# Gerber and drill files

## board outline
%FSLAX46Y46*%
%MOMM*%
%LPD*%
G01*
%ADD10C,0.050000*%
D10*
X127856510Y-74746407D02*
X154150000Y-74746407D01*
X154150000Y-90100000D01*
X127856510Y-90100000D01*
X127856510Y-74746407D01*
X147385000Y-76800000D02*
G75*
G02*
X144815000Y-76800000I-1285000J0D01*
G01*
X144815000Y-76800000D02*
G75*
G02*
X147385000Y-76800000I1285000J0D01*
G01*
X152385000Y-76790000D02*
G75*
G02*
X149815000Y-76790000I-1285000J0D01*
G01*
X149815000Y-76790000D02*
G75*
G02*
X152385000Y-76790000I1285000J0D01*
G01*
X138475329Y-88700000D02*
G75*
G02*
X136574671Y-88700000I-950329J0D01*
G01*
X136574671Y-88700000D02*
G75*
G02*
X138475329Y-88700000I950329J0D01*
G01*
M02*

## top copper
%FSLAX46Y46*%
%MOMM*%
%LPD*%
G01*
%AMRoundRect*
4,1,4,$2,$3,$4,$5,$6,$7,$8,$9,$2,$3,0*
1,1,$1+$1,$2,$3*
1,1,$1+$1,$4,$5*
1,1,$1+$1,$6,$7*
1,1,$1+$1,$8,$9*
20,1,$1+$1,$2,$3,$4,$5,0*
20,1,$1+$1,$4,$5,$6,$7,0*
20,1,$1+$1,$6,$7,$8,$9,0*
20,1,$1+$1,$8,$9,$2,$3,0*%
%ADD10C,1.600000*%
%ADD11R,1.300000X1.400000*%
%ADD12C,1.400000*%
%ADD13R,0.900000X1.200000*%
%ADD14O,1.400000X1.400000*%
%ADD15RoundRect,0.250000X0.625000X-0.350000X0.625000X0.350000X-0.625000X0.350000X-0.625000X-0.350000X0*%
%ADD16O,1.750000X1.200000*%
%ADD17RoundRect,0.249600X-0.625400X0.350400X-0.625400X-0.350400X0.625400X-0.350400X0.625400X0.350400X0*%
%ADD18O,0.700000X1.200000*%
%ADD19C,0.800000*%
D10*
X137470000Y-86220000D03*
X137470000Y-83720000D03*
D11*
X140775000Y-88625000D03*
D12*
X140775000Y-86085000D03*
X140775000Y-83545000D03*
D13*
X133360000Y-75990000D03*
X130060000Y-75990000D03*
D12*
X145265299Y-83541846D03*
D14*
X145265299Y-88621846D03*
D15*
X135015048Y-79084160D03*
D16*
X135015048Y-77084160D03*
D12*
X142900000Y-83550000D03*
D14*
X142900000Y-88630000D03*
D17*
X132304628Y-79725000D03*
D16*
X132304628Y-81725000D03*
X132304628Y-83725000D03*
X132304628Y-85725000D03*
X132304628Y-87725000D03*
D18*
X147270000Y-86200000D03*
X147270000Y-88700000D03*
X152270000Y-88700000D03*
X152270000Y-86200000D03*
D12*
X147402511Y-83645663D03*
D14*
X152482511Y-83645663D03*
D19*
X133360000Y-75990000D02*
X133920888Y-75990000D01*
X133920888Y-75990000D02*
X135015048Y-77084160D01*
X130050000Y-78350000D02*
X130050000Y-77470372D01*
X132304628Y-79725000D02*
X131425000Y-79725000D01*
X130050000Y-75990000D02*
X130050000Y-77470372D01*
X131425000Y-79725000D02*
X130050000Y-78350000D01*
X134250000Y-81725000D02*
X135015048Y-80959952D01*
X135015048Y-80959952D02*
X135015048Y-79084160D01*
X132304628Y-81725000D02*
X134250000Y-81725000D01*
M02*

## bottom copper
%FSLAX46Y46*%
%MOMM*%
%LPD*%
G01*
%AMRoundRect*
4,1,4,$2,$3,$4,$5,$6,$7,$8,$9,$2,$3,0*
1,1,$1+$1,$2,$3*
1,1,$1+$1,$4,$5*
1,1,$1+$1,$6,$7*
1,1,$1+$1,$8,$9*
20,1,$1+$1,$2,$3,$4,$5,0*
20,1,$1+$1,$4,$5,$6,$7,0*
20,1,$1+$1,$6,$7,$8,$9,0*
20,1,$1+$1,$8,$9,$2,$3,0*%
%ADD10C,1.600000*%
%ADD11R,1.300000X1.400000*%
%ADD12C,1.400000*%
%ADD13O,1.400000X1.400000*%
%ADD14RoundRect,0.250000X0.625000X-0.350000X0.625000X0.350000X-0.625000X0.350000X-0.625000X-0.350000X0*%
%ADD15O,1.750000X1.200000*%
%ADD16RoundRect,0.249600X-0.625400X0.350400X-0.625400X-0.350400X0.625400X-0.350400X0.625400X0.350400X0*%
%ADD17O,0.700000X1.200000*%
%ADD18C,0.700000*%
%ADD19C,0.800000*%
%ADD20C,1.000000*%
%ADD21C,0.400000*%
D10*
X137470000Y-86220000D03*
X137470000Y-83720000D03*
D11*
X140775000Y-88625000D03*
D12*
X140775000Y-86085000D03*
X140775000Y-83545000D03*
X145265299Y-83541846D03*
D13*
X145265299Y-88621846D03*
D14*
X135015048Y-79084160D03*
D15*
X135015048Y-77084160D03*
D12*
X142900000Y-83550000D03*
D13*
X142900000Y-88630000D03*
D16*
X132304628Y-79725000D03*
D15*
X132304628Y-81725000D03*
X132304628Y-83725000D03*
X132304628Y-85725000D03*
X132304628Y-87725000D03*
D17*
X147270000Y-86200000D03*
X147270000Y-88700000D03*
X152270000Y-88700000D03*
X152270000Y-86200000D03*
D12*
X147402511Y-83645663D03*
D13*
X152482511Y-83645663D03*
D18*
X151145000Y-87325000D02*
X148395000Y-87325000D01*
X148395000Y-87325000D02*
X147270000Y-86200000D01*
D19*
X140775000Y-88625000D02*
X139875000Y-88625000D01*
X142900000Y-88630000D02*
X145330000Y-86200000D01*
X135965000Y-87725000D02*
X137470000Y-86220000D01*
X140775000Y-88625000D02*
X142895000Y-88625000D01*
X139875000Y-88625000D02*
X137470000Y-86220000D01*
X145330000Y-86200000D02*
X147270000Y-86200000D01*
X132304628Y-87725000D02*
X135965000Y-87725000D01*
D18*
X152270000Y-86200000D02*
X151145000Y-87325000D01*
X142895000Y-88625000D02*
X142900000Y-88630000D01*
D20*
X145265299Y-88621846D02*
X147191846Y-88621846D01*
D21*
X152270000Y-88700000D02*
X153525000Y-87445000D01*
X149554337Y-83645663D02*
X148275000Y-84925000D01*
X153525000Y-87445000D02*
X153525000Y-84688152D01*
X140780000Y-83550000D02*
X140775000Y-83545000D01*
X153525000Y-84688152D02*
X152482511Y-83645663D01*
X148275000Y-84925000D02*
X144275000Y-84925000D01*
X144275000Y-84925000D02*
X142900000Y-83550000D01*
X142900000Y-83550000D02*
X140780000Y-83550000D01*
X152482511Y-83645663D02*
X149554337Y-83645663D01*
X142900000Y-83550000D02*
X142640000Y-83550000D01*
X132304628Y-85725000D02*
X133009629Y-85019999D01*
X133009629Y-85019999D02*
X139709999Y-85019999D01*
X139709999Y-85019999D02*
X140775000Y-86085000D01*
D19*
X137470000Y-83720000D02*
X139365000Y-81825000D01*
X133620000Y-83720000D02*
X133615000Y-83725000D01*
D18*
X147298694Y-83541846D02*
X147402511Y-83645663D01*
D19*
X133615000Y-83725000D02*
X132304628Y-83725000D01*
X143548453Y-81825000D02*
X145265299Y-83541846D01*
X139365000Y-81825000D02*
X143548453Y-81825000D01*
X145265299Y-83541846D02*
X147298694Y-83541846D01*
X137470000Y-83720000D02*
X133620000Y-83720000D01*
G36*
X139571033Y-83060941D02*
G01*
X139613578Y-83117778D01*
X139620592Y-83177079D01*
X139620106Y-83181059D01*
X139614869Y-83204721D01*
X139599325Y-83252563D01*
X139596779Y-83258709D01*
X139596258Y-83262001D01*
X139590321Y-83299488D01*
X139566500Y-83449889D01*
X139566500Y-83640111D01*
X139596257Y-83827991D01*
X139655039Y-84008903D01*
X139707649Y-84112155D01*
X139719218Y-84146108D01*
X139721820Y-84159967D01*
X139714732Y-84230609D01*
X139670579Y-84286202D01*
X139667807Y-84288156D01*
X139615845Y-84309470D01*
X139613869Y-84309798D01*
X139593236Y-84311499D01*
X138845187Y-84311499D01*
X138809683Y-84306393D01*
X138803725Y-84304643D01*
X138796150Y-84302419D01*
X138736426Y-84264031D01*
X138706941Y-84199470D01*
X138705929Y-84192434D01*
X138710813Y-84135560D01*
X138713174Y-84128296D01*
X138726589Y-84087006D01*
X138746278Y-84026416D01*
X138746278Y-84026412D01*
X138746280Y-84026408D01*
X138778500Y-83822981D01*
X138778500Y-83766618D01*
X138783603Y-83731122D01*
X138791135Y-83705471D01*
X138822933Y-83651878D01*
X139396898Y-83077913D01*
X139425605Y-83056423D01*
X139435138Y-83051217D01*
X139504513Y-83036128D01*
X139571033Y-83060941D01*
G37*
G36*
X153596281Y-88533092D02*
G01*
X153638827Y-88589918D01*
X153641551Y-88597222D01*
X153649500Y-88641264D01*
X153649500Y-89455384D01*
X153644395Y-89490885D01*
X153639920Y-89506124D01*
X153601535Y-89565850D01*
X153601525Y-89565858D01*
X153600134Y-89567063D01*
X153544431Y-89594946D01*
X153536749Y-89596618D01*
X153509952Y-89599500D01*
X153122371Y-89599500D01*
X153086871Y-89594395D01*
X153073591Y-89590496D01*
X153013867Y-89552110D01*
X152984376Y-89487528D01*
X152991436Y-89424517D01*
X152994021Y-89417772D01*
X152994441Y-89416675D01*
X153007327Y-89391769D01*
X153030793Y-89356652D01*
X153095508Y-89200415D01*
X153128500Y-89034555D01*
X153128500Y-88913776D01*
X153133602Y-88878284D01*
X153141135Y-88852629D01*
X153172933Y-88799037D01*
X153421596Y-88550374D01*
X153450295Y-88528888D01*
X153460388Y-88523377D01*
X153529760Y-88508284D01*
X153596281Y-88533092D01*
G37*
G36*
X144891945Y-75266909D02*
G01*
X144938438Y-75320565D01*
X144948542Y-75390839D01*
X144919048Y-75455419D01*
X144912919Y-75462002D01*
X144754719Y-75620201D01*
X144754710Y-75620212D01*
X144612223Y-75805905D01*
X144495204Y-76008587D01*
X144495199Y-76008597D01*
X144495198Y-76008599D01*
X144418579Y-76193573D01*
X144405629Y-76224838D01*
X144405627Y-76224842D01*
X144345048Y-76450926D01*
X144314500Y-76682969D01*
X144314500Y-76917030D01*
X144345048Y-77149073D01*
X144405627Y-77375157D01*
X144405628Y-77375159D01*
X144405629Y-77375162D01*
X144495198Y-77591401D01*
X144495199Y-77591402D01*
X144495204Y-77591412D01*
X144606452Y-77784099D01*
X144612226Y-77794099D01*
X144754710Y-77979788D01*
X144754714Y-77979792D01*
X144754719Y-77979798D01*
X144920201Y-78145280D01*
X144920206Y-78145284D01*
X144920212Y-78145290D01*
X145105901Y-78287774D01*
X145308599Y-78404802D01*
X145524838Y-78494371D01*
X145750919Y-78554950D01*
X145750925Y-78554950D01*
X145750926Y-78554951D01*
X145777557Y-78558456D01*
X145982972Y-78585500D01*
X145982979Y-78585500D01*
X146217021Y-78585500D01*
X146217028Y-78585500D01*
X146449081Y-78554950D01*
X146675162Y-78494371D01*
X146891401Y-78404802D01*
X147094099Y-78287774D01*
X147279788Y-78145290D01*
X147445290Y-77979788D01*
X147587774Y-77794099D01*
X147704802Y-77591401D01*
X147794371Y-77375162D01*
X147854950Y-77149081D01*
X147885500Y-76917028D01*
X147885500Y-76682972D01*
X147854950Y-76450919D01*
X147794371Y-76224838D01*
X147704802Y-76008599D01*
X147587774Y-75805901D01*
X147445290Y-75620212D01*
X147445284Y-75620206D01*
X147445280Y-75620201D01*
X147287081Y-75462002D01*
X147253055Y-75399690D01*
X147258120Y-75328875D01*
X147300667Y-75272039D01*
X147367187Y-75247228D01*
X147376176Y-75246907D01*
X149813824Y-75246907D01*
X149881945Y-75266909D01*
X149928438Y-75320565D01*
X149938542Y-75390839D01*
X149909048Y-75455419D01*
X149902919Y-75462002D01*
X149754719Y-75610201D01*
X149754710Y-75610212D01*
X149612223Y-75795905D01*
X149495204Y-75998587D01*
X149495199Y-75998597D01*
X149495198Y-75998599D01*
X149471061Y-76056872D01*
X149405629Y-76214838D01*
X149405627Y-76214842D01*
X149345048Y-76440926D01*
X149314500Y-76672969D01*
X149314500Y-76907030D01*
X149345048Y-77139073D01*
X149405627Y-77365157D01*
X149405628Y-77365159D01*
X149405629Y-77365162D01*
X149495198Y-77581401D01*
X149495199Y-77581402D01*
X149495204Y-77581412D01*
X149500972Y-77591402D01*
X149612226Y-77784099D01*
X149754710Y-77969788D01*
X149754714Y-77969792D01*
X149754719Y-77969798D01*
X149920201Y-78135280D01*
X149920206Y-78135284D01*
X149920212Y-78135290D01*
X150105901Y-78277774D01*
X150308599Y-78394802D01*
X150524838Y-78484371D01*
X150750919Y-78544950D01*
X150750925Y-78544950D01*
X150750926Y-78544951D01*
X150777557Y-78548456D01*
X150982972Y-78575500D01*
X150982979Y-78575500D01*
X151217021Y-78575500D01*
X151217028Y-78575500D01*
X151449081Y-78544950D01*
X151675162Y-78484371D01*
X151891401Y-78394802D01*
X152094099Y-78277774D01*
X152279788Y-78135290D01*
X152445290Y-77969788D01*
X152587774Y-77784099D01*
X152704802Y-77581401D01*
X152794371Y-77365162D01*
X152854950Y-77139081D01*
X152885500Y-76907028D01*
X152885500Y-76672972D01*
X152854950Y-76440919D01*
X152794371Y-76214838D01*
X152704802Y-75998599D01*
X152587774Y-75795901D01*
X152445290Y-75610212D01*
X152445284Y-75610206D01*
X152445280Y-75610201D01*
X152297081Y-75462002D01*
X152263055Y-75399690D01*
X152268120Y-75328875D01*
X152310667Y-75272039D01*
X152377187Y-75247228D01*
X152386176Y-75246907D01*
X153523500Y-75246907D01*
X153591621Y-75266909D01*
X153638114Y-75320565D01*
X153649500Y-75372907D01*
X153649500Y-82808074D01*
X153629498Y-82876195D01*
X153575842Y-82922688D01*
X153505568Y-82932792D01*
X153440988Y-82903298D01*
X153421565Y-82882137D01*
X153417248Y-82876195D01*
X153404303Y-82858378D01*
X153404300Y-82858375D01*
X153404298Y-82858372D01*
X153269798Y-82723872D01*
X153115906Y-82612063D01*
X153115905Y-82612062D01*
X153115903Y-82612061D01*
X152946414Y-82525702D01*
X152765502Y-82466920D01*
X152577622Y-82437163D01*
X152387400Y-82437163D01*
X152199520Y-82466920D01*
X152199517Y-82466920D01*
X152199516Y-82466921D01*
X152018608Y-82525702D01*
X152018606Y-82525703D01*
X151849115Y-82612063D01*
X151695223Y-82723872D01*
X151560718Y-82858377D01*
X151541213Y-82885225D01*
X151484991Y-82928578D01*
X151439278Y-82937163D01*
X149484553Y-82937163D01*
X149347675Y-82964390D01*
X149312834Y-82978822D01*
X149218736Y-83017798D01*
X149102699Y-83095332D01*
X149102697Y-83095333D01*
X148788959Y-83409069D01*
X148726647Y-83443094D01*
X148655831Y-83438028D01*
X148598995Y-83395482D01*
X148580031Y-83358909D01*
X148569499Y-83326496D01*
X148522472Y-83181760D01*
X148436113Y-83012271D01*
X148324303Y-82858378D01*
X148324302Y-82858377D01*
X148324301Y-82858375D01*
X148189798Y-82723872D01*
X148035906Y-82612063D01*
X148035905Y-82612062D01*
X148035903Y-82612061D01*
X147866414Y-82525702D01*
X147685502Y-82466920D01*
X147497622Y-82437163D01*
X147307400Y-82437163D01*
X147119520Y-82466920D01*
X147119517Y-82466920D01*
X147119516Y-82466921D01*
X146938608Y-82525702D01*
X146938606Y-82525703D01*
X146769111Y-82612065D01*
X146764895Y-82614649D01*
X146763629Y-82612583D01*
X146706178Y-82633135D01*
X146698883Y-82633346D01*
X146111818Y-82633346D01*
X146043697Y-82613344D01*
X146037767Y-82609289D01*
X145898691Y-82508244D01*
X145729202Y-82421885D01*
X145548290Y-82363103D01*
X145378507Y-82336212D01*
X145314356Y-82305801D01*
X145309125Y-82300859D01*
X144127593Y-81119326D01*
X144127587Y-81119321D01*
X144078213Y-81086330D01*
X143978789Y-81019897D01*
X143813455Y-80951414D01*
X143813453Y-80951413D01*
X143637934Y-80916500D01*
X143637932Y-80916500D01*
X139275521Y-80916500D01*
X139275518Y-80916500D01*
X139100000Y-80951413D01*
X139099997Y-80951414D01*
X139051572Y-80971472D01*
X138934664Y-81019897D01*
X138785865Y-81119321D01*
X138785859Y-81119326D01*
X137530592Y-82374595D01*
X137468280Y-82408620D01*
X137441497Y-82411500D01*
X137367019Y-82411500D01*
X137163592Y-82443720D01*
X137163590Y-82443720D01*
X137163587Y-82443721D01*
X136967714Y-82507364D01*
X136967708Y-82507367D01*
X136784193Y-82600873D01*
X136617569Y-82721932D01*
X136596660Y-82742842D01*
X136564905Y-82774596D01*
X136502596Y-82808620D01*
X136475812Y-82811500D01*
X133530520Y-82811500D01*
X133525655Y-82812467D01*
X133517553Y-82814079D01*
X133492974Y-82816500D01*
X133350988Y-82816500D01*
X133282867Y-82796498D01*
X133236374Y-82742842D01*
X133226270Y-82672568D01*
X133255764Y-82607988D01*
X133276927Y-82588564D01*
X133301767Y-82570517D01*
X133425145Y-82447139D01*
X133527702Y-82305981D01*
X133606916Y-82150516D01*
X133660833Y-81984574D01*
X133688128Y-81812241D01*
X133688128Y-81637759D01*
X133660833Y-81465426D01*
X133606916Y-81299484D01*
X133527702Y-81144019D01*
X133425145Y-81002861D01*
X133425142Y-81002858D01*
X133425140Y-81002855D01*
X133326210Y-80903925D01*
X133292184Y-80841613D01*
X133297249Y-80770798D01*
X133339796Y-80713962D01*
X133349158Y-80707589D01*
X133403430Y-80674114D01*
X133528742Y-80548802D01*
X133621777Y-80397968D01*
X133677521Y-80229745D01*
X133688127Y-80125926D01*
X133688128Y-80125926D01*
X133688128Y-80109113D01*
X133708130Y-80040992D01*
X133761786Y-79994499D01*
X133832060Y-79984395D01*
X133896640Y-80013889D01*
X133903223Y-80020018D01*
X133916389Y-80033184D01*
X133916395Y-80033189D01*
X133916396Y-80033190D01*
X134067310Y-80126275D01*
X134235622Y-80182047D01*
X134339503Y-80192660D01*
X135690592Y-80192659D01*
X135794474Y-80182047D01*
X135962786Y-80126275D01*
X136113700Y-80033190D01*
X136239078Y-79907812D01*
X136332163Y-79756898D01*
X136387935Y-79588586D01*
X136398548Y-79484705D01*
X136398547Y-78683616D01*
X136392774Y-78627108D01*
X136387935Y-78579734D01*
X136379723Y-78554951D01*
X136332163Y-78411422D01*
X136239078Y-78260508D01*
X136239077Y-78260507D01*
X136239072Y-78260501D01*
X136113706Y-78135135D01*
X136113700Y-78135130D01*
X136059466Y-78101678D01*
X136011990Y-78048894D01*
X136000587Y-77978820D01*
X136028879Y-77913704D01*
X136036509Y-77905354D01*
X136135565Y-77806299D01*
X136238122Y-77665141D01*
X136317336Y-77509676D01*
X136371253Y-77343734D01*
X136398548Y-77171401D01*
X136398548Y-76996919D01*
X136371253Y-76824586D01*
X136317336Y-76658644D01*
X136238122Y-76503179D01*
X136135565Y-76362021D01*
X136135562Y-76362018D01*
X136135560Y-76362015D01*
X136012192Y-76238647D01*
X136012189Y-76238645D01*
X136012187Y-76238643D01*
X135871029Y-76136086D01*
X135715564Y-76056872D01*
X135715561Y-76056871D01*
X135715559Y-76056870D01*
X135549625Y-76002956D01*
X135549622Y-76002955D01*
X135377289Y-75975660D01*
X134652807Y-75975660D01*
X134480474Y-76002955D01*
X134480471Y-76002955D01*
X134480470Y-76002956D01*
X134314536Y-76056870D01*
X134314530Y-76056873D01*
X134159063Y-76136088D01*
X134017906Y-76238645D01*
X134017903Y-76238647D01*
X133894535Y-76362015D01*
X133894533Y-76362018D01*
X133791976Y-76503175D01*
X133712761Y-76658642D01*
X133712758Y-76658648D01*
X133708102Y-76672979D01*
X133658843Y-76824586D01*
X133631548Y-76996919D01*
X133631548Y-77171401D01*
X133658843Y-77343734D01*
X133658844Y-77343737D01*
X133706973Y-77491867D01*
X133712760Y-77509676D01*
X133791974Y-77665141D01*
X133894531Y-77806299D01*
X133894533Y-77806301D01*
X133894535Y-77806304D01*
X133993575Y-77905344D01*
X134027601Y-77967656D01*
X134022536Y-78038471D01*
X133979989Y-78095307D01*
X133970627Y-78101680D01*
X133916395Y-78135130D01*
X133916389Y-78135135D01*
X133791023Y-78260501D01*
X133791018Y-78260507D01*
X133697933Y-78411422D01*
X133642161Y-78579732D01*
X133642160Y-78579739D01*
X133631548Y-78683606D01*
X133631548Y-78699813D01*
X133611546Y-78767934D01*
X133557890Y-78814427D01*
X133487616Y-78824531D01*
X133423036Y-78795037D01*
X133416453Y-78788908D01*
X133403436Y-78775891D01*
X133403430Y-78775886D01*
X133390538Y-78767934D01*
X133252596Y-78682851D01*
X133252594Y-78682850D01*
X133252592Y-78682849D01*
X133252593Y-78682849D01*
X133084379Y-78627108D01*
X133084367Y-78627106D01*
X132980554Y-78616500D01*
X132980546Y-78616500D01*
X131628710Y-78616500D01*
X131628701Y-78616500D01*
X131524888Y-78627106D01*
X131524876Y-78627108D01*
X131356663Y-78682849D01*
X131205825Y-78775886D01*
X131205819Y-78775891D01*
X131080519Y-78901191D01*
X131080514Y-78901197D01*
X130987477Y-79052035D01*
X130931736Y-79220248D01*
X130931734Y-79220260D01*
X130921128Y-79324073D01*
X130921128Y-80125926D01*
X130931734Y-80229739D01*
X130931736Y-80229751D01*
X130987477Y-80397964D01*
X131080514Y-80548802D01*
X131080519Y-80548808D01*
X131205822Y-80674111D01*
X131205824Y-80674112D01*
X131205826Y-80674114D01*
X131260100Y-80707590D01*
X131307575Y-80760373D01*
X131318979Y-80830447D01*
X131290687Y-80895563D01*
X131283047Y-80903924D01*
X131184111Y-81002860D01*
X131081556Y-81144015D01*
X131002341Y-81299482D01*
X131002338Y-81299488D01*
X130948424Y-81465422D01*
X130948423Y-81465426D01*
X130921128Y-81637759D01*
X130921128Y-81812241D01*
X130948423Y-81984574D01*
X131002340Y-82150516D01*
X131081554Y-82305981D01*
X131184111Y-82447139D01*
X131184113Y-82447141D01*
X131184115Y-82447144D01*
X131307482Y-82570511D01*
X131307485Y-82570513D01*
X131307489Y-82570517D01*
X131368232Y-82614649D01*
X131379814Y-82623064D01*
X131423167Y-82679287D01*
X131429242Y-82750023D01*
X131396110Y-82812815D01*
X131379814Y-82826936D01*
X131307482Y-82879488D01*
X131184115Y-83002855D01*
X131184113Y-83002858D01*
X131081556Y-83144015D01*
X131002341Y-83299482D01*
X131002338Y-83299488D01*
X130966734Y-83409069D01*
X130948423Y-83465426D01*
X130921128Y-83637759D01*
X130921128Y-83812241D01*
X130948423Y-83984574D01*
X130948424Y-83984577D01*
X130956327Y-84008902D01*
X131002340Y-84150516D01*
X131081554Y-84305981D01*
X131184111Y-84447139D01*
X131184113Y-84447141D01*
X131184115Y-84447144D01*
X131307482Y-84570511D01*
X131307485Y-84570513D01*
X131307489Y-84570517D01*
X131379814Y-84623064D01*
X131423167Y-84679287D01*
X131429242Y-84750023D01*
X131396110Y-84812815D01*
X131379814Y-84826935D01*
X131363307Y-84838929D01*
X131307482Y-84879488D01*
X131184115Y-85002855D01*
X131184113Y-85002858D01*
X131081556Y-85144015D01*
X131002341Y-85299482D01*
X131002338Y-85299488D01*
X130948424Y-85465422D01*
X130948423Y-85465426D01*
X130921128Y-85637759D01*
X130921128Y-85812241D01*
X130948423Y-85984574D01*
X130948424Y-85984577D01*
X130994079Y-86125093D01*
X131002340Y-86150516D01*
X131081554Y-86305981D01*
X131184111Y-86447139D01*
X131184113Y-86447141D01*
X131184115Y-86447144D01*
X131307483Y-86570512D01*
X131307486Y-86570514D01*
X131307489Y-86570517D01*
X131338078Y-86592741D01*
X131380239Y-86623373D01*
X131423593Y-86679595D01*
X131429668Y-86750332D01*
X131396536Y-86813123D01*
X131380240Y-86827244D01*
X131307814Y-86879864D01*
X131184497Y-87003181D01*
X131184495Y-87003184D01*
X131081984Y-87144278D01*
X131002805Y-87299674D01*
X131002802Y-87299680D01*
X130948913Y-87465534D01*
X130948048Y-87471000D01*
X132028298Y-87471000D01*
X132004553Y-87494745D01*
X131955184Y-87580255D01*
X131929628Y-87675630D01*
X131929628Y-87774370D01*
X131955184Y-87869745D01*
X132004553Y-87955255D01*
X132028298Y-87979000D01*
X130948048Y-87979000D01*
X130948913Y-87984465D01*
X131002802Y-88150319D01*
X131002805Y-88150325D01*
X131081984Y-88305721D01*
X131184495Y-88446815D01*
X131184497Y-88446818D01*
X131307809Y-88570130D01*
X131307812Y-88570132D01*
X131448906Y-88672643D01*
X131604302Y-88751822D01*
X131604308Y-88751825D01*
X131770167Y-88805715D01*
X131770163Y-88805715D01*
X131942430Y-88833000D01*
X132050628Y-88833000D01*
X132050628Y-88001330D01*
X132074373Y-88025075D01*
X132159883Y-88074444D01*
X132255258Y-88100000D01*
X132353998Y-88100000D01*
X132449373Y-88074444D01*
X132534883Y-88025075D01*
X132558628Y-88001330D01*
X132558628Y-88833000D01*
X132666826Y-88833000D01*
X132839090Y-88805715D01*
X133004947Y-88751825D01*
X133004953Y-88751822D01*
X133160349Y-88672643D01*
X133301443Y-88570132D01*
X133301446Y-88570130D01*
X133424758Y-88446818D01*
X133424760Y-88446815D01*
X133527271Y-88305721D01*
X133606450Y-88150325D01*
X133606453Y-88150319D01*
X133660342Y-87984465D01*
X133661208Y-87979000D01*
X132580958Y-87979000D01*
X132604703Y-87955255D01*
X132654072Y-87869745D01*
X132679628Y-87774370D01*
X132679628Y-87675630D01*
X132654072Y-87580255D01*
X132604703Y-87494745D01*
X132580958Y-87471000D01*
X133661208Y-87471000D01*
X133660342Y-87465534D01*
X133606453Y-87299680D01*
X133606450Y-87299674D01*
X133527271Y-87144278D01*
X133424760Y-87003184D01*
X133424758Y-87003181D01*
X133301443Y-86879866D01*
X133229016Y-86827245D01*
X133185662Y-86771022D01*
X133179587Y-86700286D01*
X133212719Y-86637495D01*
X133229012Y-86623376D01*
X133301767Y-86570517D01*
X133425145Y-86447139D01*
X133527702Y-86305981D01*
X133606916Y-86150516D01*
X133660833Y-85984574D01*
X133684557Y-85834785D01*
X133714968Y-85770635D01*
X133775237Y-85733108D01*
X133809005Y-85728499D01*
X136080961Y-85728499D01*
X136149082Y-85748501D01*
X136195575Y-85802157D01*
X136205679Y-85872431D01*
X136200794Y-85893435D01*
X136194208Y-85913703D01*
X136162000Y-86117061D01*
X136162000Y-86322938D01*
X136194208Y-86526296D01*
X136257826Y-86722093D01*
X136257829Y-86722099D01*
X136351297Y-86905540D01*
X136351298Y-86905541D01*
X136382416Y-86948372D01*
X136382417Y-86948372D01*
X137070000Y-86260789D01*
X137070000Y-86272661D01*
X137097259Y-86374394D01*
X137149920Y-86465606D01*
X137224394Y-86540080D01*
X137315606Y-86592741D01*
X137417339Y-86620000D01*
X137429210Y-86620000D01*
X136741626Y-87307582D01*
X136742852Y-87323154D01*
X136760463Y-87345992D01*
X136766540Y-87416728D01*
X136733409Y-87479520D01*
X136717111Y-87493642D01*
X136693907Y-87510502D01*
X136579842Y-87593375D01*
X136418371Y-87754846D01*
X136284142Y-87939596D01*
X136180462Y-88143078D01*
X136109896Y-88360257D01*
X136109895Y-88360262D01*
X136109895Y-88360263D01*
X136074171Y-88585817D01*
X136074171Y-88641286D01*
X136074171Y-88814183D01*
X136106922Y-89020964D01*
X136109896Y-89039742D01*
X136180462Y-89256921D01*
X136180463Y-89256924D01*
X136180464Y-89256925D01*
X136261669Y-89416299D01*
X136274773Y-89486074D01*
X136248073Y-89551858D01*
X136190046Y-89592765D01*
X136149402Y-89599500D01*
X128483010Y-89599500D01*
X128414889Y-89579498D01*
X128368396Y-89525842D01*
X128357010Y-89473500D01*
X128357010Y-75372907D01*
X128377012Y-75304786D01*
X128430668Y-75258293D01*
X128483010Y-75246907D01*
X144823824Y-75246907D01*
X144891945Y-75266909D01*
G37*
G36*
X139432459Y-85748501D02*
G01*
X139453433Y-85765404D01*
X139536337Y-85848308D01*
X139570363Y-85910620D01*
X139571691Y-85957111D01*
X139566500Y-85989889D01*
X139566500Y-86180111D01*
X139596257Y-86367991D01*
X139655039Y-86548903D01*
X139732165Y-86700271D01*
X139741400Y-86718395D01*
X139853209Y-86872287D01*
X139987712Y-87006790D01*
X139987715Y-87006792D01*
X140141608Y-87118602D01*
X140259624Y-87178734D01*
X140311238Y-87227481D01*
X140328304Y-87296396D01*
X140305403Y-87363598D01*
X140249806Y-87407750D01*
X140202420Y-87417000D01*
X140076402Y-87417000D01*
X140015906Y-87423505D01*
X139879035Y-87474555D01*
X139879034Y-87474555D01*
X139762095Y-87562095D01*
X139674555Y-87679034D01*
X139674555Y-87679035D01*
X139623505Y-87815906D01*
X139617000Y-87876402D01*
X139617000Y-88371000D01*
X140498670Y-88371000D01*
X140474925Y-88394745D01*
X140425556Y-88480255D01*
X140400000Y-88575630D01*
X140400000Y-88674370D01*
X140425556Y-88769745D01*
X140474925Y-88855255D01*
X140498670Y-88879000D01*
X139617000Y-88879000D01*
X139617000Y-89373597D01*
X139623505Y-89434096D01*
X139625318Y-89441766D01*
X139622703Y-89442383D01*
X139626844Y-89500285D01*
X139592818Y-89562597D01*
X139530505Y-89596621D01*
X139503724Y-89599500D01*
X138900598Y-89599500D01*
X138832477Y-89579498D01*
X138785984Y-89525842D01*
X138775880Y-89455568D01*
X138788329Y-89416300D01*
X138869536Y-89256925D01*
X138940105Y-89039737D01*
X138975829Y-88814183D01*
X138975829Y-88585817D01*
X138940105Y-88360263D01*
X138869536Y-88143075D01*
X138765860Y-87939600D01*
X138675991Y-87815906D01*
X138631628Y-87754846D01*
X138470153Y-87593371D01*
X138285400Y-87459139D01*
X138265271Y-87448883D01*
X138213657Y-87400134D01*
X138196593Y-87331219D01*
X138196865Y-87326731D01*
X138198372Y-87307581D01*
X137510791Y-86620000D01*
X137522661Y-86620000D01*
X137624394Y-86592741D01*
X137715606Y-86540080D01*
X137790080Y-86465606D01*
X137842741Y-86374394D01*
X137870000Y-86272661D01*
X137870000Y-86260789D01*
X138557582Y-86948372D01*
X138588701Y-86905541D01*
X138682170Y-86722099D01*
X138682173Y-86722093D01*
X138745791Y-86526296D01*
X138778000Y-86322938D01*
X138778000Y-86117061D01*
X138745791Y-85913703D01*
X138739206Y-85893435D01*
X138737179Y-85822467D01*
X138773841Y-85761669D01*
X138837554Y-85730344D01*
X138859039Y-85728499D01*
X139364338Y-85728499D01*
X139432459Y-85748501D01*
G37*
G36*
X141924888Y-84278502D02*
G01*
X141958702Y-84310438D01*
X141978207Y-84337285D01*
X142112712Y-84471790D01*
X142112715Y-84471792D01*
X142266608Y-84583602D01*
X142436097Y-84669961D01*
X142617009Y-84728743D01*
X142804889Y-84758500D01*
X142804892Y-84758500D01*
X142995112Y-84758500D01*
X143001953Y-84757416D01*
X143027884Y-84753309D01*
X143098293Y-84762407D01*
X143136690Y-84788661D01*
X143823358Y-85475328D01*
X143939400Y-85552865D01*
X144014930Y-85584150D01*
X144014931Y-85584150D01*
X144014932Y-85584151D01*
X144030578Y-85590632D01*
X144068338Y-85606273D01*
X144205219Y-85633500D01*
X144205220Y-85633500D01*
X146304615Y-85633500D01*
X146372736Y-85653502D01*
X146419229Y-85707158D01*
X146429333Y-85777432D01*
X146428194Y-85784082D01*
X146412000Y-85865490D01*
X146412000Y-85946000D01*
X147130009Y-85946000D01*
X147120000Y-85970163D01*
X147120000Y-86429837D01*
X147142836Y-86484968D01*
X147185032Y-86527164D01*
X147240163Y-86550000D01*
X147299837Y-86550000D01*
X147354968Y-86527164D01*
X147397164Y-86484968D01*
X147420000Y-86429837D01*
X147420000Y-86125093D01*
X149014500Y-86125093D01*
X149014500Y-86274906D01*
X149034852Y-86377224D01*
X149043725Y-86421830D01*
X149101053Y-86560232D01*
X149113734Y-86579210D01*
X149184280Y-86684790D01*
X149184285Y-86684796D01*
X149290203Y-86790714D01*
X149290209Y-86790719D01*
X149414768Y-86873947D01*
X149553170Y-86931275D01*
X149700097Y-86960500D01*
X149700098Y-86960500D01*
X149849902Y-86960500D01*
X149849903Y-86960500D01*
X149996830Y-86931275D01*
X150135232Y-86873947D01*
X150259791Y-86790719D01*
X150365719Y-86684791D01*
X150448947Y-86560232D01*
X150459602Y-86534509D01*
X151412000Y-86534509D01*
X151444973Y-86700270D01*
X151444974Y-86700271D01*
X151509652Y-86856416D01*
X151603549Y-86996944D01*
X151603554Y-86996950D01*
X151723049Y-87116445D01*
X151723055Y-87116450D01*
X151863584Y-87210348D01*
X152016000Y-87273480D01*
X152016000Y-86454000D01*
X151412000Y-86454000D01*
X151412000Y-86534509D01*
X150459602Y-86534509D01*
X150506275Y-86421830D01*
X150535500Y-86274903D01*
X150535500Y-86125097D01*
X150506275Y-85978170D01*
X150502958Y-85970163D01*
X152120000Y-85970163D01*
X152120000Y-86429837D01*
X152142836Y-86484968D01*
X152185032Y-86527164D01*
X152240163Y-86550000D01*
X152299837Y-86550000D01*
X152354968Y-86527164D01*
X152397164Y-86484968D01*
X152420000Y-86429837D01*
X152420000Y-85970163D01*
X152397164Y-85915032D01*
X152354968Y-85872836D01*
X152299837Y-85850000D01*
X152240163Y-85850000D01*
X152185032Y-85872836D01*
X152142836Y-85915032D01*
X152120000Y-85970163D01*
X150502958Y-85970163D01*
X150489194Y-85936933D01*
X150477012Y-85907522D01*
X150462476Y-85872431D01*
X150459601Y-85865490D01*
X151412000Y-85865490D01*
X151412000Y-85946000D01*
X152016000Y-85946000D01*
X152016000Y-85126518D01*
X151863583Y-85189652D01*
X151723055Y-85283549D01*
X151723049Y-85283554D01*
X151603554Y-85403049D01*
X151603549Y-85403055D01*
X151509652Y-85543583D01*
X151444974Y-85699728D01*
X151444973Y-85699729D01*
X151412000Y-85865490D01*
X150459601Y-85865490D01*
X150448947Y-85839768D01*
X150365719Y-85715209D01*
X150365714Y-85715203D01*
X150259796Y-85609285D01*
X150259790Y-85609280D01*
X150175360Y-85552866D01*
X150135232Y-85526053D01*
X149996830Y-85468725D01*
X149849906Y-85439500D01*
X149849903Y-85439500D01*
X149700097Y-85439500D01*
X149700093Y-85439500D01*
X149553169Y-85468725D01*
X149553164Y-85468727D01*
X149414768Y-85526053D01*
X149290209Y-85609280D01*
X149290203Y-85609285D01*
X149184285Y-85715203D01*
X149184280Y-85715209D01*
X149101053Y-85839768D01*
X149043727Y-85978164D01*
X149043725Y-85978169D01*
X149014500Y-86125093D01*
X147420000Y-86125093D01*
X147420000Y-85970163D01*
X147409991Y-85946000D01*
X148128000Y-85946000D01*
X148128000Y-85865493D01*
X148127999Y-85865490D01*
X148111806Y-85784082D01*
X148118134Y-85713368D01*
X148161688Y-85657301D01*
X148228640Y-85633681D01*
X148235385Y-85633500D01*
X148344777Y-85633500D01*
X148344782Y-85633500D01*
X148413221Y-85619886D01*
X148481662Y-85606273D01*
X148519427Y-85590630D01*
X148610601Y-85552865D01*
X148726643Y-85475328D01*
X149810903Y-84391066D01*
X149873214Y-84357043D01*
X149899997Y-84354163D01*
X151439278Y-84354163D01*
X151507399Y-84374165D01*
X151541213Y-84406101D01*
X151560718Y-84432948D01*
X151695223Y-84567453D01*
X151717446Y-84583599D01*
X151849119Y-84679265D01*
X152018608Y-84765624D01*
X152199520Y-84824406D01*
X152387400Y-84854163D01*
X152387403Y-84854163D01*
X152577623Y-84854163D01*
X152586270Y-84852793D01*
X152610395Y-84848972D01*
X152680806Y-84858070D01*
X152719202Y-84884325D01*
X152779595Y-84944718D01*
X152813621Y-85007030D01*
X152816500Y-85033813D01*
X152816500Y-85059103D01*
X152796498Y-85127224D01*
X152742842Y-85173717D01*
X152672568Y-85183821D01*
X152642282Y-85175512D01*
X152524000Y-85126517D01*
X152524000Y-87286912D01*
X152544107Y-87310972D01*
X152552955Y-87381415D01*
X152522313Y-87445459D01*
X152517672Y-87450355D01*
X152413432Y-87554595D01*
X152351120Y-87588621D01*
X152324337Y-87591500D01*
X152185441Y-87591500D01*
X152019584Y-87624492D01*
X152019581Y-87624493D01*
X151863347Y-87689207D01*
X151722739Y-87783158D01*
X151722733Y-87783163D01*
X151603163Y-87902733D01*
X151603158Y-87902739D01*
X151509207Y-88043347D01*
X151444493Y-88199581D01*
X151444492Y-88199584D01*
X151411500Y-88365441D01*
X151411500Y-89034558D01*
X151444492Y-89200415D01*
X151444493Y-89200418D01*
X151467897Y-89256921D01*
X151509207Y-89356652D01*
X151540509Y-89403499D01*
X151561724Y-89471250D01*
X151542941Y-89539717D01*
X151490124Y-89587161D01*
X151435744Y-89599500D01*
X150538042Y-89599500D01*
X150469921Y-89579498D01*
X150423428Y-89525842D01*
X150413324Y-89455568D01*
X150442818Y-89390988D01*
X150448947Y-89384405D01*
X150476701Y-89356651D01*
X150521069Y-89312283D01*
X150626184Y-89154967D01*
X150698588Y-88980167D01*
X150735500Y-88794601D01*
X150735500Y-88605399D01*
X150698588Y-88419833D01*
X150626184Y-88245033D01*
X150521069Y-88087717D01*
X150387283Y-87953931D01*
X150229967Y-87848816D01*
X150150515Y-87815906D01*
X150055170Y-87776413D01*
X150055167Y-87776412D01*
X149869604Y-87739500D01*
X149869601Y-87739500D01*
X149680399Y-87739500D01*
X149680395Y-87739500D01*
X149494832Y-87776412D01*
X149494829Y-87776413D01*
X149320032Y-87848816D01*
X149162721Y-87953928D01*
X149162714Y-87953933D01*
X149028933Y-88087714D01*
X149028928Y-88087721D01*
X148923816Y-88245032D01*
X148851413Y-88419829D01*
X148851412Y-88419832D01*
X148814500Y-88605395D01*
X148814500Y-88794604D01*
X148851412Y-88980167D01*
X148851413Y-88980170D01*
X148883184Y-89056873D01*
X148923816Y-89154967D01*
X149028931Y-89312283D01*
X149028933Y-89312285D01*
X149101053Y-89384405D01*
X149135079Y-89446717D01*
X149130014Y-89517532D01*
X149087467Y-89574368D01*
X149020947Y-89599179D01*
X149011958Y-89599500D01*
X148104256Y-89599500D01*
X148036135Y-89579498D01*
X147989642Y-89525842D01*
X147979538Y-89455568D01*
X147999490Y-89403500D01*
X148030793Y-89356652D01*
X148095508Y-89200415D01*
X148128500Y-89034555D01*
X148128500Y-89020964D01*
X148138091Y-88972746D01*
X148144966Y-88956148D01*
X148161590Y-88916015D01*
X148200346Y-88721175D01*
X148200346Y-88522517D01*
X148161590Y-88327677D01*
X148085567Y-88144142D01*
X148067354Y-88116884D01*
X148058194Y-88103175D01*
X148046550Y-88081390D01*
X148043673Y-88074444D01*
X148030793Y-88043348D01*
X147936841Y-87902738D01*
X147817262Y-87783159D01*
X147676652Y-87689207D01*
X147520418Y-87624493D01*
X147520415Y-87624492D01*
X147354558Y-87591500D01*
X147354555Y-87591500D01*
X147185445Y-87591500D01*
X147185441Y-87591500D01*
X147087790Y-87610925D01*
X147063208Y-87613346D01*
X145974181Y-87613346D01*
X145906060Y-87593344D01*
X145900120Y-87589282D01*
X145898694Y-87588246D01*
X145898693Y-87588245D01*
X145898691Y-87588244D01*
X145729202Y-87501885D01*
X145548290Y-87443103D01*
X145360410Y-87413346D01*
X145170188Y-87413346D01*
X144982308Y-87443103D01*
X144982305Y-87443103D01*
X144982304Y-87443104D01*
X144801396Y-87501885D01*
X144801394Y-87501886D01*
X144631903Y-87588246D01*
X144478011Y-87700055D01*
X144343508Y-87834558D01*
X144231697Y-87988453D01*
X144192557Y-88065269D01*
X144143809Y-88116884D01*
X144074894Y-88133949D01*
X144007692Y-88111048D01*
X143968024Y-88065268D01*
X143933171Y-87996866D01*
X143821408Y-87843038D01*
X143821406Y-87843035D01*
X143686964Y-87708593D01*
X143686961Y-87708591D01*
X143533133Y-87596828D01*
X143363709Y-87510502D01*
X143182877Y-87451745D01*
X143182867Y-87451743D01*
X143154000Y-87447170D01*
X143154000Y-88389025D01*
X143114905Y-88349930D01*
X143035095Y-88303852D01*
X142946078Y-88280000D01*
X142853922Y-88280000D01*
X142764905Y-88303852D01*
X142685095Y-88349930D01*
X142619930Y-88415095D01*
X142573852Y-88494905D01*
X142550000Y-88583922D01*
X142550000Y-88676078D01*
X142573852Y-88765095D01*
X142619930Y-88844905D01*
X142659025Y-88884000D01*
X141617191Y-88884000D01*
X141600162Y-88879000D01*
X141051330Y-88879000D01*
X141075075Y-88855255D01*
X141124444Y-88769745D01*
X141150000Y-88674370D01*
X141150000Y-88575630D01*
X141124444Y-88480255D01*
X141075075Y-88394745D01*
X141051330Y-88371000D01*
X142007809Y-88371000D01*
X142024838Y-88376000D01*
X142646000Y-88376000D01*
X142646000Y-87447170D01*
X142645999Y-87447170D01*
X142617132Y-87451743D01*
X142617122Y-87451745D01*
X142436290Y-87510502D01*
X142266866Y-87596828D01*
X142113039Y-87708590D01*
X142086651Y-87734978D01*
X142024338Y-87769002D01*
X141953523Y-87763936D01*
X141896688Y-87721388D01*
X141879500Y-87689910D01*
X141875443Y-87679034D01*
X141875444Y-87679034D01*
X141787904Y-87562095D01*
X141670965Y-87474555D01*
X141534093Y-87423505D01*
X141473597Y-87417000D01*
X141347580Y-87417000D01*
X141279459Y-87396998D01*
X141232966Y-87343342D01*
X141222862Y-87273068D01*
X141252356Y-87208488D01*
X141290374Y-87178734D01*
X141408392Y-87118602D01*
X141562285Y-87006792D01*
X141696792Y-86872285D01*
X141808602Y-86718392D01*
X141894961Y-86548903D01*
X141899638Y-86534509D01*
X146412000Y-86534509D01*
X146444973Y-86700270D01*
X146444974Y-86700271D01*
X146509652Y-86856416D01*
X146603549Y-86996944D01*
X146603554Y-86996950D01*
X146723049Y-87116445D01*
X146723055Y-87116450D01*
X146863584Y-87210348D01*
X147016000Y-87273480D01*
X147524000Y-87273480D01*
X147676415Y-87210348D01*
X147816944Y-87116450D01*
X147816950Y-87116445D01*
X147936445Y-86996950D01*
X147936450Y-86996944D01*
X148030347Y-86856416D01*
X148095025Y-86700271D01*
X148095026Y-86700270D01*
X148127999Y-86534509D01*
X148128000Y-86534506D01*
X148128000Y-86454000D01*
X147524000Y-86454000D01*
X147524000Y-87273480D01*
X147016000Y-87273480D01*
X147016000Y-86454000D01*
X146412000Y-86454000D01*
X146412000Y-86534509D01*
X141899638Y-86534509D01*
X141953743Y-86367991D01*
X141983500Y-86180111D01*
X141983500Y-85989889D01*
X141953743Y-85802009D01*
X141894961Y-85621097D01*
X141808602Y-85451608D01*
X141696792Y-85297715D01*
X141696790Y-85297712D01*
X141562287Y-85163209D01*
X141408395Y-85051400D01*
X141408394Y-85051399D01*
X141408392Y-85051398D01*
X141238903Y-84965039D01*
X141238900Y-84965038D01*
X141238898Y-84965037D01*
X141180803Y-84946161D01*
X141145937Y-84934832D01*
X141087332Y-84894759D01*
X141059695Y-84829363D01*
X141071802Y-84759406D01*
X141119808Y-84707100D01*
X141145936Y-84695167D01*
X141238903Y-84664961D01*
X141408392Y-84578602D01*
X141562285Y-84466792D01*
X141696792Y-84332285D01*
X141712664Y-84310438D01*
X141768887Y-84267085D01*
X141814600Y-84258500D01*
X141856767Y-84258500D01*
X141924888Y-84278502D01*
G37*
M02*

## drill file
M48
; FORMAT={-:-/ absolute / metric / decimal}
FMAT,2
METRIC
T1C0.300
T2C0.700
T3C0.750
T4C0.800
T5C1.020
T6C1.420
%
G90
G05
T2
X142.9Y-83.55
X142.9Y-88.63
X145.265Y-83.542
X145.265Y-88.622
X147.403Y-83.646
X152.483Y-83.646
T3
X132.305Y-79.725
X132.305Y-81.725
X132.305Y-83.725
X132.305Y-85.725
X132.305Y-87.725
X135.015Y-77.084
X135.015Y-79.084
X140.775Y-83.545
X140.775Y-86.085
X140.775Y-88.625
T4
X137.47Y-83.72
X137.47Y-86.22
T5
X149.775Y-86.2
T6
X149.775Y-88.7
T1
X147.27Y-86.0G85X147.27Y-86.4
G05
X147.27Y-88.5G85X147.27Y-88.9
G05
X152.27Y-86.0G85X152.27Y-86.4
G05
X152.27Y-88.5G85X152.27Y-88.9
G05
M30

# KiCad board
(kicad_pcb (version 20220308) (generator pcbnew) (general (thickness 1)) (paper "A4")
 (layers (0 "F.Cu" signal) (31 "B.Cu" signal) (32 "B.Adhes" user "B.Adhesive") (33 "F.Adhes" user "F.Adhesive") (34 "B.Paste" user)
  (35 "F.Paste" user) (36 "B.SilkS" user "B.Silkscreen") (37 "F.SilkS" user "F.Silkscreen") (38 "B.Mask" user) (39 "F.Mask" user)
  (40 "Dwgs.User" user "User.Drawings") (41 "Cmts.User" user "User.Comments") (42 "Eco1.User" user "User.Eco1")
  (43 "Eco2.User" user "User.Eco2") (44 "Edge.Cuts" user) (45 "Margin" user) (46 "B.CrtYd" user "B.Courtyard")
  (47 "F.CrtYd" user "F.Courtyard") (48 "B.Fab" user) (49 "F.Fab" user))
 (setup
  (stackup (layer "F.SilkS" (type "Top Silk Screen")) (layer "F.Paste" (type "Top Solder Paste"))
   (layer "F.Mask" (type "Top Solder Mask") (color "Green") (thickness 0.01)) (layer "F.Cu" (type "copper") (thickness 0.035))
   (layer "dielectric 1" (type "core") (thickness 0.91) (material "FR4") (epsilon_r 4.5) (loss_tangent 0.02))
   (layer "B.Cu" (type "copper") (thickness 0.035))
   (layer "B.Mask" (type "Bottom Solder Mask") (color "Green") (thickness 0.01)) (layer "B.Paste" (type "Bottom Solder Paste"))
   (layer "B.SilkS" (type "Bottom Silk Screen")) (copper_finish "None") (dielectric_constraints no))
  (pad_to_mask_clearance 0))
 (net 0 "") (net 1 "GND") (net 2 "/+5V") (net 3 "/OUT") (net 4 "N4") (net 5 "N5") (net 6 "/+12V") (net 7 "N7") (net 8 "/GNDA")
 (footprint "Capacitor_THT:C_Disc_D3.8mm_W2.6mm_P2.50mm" (layer "F.Cu") (at 137.47 86.22 90)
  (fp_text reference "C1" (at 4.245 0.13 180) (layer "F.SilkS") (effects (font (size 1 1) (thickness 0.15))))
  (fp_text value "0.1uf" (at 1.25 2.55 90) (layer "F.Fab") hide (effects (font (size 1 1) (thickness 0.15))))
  (pad "1" thru_hole circle locked (at 0 0 90) (size 1.6 1.6) (drill 0.8) (layers *.Cu *.Mask) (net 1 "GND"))
  (pad "2" thru_hole circle locked (at 2.5 0 90) (size 1.6 1.6) (drill 0.8) (layers *.Cu *.Mask) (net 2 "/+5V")))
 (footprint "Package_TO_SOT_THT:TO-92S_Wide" (layer "F.Cu") (at 140.775 88.625 90)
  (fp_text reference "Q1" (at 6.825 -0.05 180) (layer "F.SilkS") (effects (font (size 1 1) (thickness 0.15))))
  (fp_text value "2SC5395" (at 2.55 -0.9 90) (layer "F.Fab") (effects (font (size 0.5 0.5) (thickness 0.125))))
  (pad "1" thru_hole rect locked (at 0 0 90) (size 1.4 1.3) (drill 0.75) (layers *.Cu *.Mask) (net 1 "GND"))
  (pad "2" thru_hole circle locked (at 2.54 0 90) (size 1.4 1.4) (drill 0.75) (layers *.Cu *.Mask) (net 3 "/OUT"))
  (pad "3" thru_hole circle locked (at 5.08 0 90) (size 1.4 1.4) (drill 0.75) (layers *.Cu *.Mask) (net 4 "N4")))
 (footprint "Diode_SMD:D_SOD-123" (layer "F.Cu") (at 131.71 75.99 180)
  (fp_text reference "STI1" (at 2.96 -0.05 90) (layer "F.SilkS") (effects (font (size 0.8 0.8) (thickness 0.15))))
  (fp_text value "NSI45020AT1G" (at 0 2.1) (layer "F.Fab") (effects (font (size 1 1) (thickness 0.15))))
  (pad "1" smd rect locked (at -1.65 0 180) (size 0.9 1.2) (layers "F.Cu" "F.Paste" "F.Mask") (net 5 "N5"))
  (pad "2" smd rect locked (at 1.65 0 180) (size 0.9 1.2) (layers "F.Cu" "F.Paste" "F.Mask") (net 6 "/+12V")))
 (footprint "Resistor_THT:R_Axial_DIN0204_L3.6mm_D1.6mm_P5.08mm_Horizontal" (layer "F.Cu") (at 145.265299 83.541846 -90)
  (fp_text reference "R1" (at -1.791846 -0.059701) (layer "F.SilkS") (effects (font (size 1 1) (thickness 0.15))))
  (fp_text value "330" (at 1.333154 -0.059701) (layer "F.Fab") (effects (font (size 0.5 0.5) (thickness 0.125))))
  (pad "1" thru_hole circle locked (at 0 0 270) (size 1.4 1.4) (drill 0.7) (layers *.Cu *.Mask) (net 2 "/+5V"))
  (pad "2" thru_hole oval locked (at 5.08 0 270) (size 1.4 1.4) (drill 0.7) (layers *.Cu *.Mask) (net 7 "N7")))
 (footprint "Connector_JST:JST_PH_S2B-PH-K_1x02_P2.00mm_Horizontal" (layer "F.Cu") (at 135.015048 79.08416 90)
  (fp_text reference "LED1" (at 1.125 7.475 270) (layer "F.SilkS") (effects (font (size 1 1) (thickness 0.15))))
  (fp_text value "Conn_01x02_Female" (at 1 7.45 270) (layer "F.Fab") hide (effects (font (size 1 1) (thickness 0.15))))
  (pad "1" thru_hole roundrect locked (at 0 0 90) (size 1.2 1.75) (drill 0.75) (layers *.Cu *.Mask) (roundrect_rratio 0.2083333333)
   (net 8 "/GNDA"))
  (pad "2" thru_hole oval locked (at 2 0 90) (size 1.2 1.75) (drill 0.75) (layers *.Cu *.Mask) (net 5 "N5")))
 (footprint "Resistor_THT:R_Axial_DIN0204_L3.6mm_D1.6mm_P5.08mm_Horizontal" (layer "F.Cu") (at 142.9 83.55 -90)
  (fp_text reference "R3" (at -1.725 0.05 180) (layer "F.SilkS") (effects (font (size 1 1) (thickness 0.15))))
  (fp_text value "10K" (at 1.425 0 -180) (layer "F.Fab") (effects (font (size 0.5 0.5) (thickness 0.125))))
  (pad "1" thru_hole circle locked (at 0 0 270) (size 1.4 1.4) (drill 0.7) (layers *.Cu *.Mask) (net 4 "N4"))
  (pad "2" thru_hole oval locked (at 5.08 0 270) (size 1.4 1.4) (drill 0.7) (layers *.Cu *.Mask) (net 1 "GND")))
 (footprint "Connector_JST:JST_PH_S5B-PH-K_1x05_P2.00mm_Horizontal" (layer "F.Cu") (at 132.304628 79.725 -90)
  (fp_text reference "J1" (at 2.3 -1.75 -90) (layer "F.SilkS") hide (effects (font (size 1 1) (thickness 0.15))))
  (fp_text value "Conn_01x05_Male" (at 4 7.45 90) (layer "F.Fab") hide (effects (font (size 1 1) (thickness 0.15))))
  (pad "1" thru_hole roundrect locked (at 0 0 270) (size 1.2 1.75) (drill 0.75) (layers *.Cu *.Mask) (roundrect_rratio 0.208)
   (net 6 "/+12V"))
  (pad "2" thru_hole oval locked (at 2 0 270) (size 1.2 1.75) (drill 0.75) (layers *.Cu *.Mask) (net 8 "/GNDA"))
  (pad "3" thru_hole oval locked (at 4 0 270) (size 1.2 1.75) (drill 0.75) (layers *.Cu *.Mask) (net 2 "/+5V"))
  (pad "4" thru_hole oval locked (at 6 0 270) (size 1.2 1.75) (drill 0.75) (layers *.Cu *.Mask) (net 3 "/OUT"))
  (pad "5" thru_hole oval locked (at 8 0 270) (size 1.2 1.75) (drill 0.75) (layers *.Cu *.Mask) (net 1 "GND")))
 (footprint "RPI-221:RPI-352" (layer "F.Cu") (at 146.5 89.6)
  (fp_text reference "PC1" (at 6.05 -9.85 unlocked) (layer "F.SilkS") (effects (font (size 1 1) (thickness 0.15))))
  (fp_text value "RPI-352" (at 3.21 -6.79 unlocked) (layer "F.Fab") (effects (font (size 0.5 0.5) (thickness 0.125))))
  (pad "" np_thru_hole circle (at 3.275 -3.4) (size 1.02 1.02) (drill 1.02) (layers *.Mask))
  (pad "" np_thru_hole circle (at 3.275 -0.9) (size 1.42 1.42) (drill 1.42) (layers *.Mask))
  (pad "1" thru_hole oval (at 0.77 -3.4) (size 0.7 1.2) (drill oval 0.3 0.7) (layers *.Cu *.Mask) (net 1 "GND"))
  (pad "2" thru_hole oval (at 0.77 -0.9) (size 0.7 1.2) (drill oval 0.3 0.7) (layers *.Cu *.Mask) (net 7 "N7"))
  (pad "3" thru_hole oval (at 5.77 -0.9) (size 0.7 1.2) (drill oval 0.3 0.7) (layers *.Cu *.Mask) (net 4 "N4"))
  (pad "4" thru_hole oval (at 5.77 -3.4) (size 0.7 1.2) (drill oval 0.3 0.7) (layers *.Cu *.Mask) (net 1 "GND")))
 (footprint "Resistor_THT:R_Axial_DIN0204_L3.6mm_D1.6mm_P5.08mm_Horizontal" (layer "F.Cu") (at 147.402511 83.645663)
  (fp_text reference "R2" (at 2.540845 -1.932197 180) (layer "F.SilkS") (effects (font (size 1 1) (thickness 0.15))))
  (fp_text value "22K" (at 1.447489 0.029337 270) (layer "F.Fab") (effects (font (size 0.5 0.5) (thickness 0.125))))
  (pad "1" thru_hole circle locked (at 0 0) (size 1.4 1.4) (drill 0.7) (layers *.Cu *.Mask) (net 2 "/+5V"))
  (pad "2" thru_hole oval locked (at 5.08 0) (size 1.4 1.4) (drill 0.7) (layers *.Cu *.Mask) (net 4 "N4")))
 (gr_rect (start 127.85651 74.746407) (end 154.15 90.1) (stroke (width 0.05) (type solid)) (fill none) (layer "Edge.Cuts"))
 (gr_circle (center 146.1 76.8) (end 147.385 76.8) (stroke (width 0.05) (type solid)) (fill none) (layer "Edge.Cuts"))
 (gr_circle (center 151.1 76.79) (end 152.385 76.79) (stroke (width 0.05) (type solid)) (fill none) (layer "Edge.Cuts"))
 (gr_circle (center 137.525 88.7) (end 138.475 88.675) (stroke (width 0.05) (type solid)) (fill none) (layer "Edge.Cuts"))
 (segment (start 151.145 87.325) (end 148.395 87.325) (width 0.7) (layer "B.Cu") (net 1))
 (segment (start 148.395 87.325) (end 147.27 86.2) (width 0.7) (layer "B.Cu") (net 1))
 (segment (start 140.775 88.625) (end 139.875 88.625) (width 0.8) (layer "B.Cu") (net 1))
 (segment (start 142.9 88.63) (end 145.33 86.2) (width 0.8) (layer "B.Cu") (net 1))
 (segment (start 135.965 87.725) (end 137.47 86.22) (width 0.8) (layer "B.Cu") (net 1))
 (segment (start 140.775 88.625) (end 142.895 88.625) (width 0.8) (layer "B.Cu") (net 1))
 (segment (start 139.875 88.625) (end 137.47 86.22) (width 0.8) (layer "B.Cu") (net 1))
 (segment (start 145.33 86.2) (end 147.27 86.2) (width 0.8) (layer "B.Cu") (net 1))
 (segment (start 132.304628 87.725) (end 135.965 87.725) (width 0.8) (layer "B.Cu") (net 1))
 (segment (start 152.27 86.2) (end 151.145 87.325) (width 0.7) (layer "B.Cu") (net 1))
 (segment (start 142.895 88.625) (end 142.9 88.63) (width 0.7) (layer "B.Cu") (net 1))
 (segment (start 133.36 75.99) (end 133.920888 75.99) (width 0.8) (layer "F.Cu") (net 5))
 (segment (start 133.920888 75.99) (end 135.015048 77.08416) (width 0.8) (layer "F.Cu") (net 5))
 (segment (start 145.265299 88.621846) (end 147.191846 88.621846) (width 1) (layer "B.Cu") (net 7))
 (segment (start 152.27 88.7) (end 153.525 87.445) (width 0.4) (layer "B.Cu") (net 4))
 (segment (start 149.554337 83.645663) (end 148.275 84.925) (width 0.4) (layer "B.Cu") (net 4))
 (segment (start 153.525 87.445) (end 153.525 84.688152) (width 0.4) (layer "B.Cu") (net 4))
 (segment (start 140.78 83.55) (end 140.775 83.545) (width 0.4) (layer "B.Cu") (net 4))
 (segment (start 153.525 84.688152) (end 152.482511 83.645663) (width 0.4) (layer "B.Cu") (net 4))
 (segment (start 148.275 84.925) (end 144.275 84.925) (width 0.4) (layer "B.Cu") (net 4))
 (segment (start 144.275 84.925) (end 142.9 83.55) (width 0.4) (layer "B.Cu") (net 4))
 (segment (start 142.9 83.55) (end 140.78 83.55) (width 0.4) (layer "B.Cu") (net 4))
 (segment (start 152.482511 83.645663) (end 149.554337 83.645663) (width 0.4) (layer "B.Cu") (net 4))
 (segment (start 142.9 83.55) (end 142.64 83.55) (width 0.4) (layer "B.Cu") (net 4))
 (segment (start 132.304628 85.725) (end 133.009629 85.019999) (width 0.4) (layer "B.Cu") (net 3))
 (segment (start 133.009629 85.019999) (end 139.709999 85.019999) (width 0.4) (layer "B.Cu") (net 3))
 (segment (start 139.709999 85.019999) (end 140.775 86.085) (width 0.4) (layer "B.Cu") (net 3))
 (segment (start 130.05 78.35) (end 130.05 77.470372) (width 0.8) (layer "F.Cu") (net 6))
 (segment (start 132.304628 79.725) (end 131.425 79.725) (width 0.8) (layer "F.Cu") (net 6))
 (segment (start 130.05 75.99) (end 130.05 77.470372) (width 0.8) (layer "F.Cu") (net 6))
 (segment (start 131.425 79.725) (end 130.05 78.35) (width 0.8) (layer "F.Cu") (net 6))
 (segment (start 134.25 81.725) (end 135.015048 80.959952) (width 0.8) (layer "F.Cu") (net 8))
 (segment (start 135.015048 80.959952) (end 135.015048 79.08416) (width 0.8) (layer "F.Cu") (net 8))
 (segment (start 132.304628 81.725) (end 134.25 81.725) (width 0.8) (layer "F.Cu") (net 8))
 (segment (start 137.47 83.72) (end 139.365 81.825) (width 0.8) (layer "B.Cu") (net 2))
 (segment (start 133.62 83.72) (end 133.615 83.725) (width 0.8) (layer "B.Cu") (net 2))
 (segment (start 147.298694 83.541846) (end 147.402511 83.645663) (width 0.7) (layer "B.Cu") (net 2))
 (segment (start 133.615 83.725) (end 132.304628 83.725) (width 0.8) (layer "B.Cu") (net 2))
 (segment (start 143.548453 81.825) (end 145.265299 83.541846) (width 0.8) (layer "B.Cu") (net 2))
 (segment (start 139.365 81.825) (end 143.548453 81.825) (width 0.8) (layer "B.Cu") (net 2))
 (segment (start 145.265299 83.541846) (end 147.298694 83.541846) (width 0.8) (layer "B.Cu") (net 2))
 (segment (start 137.47 83.72) (end 133.62 83.72) (width 0.8) (layer "B.Cu") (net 2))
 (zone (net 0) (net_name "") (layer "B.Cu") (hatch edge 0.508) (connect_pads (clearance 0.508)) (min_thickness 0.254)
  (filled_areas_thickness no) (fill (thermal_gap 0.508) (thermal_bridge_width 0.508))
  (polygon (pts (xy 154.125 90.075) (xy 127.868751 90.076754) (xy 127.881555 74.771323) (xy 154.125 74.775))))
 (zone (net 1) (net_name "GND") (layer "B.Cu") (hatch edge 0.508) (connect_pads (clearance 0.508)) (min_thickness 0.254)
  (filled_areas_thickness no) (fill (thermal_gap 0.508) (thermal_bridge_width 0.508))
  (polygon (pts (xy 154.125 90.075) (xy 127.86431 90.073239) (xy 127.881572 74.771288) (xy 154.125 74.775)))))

